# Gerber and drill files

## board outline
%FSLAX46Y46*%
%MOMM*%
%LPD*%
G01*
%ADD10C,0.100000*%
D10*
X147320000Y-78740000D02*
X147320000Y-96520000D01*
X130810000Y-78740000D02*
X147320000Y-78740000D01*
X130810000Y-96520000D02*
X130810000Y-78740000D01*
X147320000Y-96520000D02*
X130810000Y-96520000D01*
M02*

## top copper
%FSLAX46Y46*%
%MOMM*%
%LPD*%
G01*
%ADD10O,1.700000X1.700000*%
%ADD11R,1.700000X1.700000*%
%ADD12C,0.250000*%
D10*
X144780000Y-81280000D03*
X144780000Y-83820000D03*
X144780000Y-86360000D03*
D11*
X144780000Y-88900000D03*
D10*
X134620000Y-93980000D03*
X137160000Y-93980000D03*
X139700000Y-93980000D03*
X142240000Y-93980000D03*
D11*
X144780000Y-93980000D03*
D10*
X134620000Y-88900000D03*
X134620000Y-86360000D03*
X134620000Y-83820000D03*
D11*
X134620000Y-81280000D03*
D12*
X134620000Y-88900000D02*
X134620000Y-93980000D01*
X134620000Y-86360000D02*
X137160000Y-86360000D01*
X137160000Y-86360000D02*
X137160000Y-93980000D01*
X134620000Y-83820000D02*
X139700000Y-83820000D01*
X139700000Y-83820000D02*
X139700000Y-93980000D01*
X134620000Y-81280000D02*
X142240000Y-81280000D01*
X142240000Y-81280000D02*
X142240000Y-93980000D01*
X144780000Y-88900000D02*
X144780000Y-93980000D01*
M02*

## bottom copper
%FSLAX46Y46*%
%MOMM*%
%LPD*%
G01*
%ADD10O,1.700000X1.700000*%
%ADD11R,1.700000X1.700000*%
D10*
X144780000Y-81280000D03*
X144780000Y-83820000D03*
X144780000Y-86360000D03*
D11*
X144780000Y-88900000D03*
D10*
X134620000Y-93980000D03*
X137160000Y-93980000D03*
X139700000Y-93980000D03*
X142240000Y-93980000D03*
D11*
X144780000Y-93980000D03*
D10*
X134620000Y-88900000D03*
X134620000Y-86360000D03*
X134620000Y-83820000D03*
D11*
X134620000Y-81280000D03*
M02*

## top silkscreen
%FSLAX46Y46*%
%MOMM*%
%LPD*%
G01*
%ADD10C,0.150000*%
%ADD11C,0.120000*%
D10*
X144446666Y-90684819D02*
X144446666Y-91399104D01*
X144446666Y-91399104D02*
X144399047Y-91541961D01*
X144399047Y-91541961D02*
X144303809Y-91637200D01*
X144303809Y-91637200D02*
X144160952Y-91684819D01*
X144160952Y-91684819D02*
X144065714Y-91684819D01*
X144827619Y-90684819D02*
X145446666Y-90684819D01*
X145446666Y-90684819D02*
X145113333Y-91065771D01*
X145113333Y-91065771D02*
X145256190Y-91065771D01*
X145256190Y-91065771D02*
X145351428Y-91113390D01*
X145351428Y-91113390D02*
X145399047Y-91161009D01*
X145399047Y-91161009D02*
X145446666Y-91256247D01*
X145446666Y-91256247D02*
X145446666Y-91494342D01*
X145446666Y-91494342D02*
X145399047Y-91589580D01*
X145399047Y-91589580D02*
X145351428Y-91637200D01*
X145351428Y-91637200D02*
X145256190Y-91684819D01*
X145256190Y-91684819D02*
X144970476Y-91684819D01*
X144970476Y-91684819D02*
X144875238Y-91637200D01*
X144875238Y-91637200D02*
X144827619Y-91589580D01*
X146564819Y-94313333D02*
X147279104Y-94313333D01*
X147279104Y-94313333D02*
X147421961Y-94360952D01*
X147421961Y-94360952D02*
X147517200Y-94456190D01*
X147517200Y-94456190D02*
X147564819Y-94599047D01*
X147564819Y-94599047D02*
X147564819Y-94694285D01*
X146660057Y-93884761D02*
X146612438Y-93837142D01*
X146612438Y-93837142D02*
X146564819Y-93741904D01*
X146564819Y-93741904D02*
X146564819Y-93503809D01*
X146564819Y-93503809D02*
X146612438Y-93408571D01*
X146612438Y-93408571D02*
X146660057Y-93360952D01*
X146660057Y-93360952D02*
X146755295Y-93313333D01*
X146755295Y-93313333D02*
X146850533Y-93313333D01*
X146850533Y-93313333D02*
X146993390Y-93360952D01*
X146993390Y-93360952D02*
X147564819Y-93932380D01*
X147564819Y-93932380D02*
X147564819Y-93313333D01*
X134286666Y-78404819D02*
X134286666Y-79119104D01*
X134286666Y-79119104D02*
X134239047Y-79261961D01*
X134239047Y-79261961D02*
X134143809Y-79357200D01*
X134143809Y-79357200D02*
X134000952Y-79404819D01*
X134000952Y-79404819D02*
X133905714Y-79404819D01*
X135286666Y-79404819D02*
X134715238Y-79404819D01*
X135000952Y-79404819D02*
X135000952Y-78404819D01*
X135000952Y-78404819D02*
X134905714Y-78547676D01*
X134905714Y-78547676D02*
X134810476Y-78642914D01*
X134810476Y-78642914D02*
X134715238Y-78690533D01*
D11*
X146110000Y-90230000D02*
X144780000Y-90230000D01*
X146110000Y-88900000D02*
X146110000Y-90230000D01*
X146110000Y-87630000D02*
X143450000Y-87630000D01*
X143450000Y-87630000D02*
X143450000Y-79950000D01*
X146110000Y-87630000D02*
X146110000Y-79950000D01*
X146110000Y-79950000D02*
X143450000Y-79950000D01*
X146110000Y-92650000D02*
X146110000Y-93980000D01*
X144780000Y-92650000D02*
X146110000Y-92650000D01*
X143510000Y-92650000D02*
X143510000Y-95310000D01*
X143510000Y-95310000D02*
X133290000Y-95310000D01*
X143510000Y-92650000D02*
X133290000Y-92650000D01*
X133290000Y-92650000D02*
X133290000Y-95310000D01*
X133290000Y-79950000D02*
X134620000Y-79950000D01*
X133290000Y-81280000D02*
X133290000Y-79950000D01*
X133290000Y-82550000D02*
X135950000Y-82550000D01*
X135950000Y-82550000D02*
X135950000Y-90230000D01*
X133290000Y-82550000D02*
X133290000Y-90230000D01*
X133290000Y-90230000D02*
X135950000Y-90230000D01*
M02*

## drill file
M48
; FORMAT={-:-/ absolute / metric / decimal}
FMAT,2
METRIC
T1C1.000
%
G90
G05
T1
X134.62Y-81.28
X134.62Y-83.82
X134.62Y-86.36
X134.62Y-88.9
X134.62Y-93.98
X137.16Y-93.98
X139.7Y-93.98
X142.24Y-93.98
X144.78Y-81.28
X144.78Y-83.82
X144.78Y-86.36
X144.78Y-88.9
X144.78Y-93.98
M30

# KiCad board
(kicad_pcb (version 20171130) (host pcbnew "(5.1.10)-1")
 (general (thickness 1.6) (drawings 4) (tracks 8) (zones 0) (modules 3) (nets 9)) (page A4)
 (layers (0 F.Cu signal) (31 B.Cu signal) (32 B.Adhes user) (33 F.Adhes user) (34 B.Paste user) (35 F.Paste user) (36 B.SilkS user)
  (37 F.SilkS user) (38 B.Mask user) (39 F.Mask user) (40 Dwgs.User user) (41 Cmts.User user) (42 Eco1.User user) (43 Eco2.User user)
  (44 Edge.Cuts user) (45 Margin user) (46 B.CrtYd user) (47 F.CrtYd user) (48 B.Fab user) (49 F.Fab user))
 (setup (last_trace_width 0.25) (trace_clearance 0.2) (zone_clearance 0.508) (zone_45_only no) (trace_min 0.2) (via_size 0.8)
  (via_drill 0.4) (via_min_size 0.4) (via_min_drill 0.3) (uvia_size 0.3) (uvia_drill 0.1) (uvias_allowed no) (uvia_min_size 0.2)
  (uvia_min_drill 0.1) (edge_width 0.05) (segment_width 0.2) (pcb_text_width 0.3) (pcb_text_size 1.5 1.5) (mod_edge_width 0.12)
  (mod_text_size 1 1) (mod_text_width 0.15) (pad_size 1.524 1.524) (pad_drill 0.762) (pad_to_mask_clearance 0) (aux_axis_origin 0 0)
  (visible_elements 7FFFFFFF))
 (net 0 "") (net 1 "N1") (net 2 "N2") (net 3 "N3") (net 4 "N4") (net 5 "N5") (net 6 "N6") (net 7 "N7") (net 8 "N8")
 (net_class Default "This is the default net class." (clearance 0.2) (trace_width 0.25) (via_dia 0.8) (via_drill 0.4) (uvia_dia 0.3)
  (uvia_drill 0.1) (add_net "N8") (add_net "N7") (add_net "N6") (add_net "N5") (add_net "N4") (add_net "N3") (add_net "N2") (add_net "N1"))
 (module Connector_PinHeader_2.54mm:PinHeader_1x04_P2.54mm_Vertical (layer F.Cu) (at 144.78 88.9 180)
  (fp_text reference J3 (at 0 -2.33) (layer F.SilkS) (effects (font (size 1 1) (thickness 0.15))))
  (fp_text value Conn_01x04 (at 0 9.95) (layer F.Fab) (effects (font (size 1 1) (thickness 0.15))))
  (fp_line (start -1.33 -1.33) (end 0 -1.33) (layer F.SilkS) (width 0.12))
  (fp_line (start -1.33 0) (end -1.33 -1.33) (layer F.SilkS) (width 0.12))
  (fp_line (start -1.33 1.27) (end 1.33 1.27) (layer F.SilkS) (width 0.12))
  (fp_line (start 1.33 1.27) (end 1.33 8.95) (layer F.SilkS) (width 0.12))
  (fp_line (start -1.33 1.27) (end -1.33 8.95) (layer F.SilkS) (width 0.12))
  (fp_line (start -1.33 8.95) (end 1.33 8.95) (layer F.SilkS) (width 0.12))
  (pad 4 thru_hole oval (at 0 7.62 180) (size 1.7 1.7) (drill 1) (layers *.Cu *.Mask) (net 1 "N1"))
  (pad 3 thru_hole oval (at 0 5.08 180) (size 1.7 1.7) (drill 1) (layers *.Cu *.Mask) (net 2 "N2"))
  (pad 2 thru_hole oval (at 0 2.54 180) (size 1.7 1.7) (drill 1) (layers *.Cu *.Mask) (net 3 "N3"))
  (pad 1 thru_hole rect (at 0 0 180) (size 1.7 1.7) (drill 1) (layers *.Cu *.Mask) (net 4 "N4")))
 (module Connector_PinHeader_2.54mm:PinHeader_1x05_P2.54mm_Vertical (layer F.Cu) (at 144.78 93.98 270)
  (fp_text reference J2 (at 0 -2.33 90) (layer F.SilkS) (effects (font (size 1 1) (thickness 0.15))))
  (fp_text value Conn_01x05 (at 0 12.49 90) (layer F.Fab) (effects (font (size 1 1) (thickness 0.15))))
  (fp_line (start -1.33 -1.33) (end 0 -1.33) (layer F.SilkS) (width 0.12))
  (fp_line (start -1.33 0) (end -1.33 -1.33) (layer F.SilkS) (width 0.12))
  (fp_line (start -1.33 1.27) (end 1.33 1.27) (layer F.SilkS) (width 0.12))
  (fp_line (start 1.33 1.27) (end 1.33 11.49) (layer F.SilkS) (width 0.12))
  (fp_line (start -1.33 1.27) (end -1.33 11.49) (layer F.SilkS) (width 0.12))
  (fp_line (start -1.33 11.49) (end 1.33 11.49) (layer F.SilkS) (width 0.12))
  (pad 5 thru_hole oval (at 0 10.16 270) (size 1.7 1.7) (drill 1) (layers *.Cu *.Mask) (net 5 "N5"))
  (pad 4 thru_hole oval (at 0 7.62 270) (size 1.7 1.7) (drill 1) (layers *.Cu *.Mask) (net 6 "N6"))
  (pad 3 thru_hole oval (at 0 5.08 270) (size 1.7 1.7) (drill 1) (layers *.Cu *.Mask) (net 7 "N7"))
  (pad 2 thru_hole oval (at 0 2.54 270) (size 1.7 1.7) (drill 1) (layers *.Cu *.Mask) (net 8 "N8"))
  (pad 1 thru_hole rect (at 0 0 270) (size 1.7 1.7) (drill 1) (layers *.Cu *.Mask) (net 4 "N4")))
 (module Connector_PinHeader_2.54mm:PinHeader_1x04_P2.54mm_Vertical (layer F.Cu) (at 134.62 81.28)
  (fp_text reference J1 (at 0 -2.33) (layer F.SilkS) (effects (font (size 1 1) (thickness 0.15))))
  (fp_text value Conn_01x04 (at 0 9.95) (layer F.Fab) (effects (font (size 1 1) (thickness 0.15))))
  (fp_line (start -1.33 -1.33) (end 0 -1.33) (layer F.SilkS) (width 0.12))
  (fp_line (start -1.33 0) (end -1.33 -1.33) (layer F.SilkS) (width 0.12))
  (fp_line (start -1.33 1.27) (end 1.33 1.27) (layer F.SilkS) (width 0.12))
  (fp_line (start 1.33 1.27) (end 1.33 8.95) (layer F.SilkS) (width 0.12))
  (fp_line (start -1.33 1.27) (end -1.33 8.95) (layer F.SilkS) (width 0.12))
  (fp_line (start -1.33 8.95) (end 1.33 8.95) (layer F.SilkS) (width 0.12))
  (pad 4 thru_hole oval (at 0 7.62) (size 1.7 1.7) (drill 1) (layers *.Cu *.Mask) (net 5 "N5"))
  (pad 3 thru_hole oval (at 0 5.08) (size 1.7 1.7) (drill 1) (layers *.Cu *.Mask) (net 6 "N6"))
  (pad 2 thru_hole oval (at 0 2.54) (size 1.7 1.7) (drill 1) (layers *.Cu *.Mask) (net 7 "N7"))
  (pad 1 thru_hole rect (at 0 0) (size 1.7 1.7) (drill 1) (layers *.Cu *.Mask) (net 8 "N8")))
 (gr_line (start 147.32 78.74) (end 147.32 96.52) (layer Edge.Cuts) (width 0.1))
 (gr_line (start 130.81 78.74) (end 147.32 78.74) (layer Edge.Cuts) (width 0.1))
 (gr_line (start 130.81 96.52) (end 130.81 78.74) (layer Edge.Cuts) (width 0.1))
 (gr_line (start 147.32 96.52) (end 130.81 96.52) (layer Edge.Cuts) (width 0.1))
 (segment (start 134.62 88.9) (end 134.62 93.98) (width 0.25) (layer F.Cu) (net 5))
 (segment (start 134.62 86.36) (end 137.16 86.36) (width 0.25) (layer F.Cu) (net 6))
 (segment (start 137.16 86.36) (end 137.16 93.98) (width 0.25) (layer F.Cu) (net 6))
 (segment (start 134.62 83.82) (end 139.7 83.82) (width 0.25) (layer F.Cu) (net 7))
 (segment (start 139.7 83.82) (end 139.7 93.98) (width 0.25) (layer F.Cu) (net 7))
 (segment (start 134.62 81.28) (end 142.24 81.28) (width 0.25) (layer F.Cu) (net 8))
 (segment (start 142.24 81.28) (end 142.24 93.98) (width 0.25) (layer F.Cu) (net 8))
 (segment (start 144.78 88.9) (end 144.78 93.98) (width 0.25) (layer F.Cu) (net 4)))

